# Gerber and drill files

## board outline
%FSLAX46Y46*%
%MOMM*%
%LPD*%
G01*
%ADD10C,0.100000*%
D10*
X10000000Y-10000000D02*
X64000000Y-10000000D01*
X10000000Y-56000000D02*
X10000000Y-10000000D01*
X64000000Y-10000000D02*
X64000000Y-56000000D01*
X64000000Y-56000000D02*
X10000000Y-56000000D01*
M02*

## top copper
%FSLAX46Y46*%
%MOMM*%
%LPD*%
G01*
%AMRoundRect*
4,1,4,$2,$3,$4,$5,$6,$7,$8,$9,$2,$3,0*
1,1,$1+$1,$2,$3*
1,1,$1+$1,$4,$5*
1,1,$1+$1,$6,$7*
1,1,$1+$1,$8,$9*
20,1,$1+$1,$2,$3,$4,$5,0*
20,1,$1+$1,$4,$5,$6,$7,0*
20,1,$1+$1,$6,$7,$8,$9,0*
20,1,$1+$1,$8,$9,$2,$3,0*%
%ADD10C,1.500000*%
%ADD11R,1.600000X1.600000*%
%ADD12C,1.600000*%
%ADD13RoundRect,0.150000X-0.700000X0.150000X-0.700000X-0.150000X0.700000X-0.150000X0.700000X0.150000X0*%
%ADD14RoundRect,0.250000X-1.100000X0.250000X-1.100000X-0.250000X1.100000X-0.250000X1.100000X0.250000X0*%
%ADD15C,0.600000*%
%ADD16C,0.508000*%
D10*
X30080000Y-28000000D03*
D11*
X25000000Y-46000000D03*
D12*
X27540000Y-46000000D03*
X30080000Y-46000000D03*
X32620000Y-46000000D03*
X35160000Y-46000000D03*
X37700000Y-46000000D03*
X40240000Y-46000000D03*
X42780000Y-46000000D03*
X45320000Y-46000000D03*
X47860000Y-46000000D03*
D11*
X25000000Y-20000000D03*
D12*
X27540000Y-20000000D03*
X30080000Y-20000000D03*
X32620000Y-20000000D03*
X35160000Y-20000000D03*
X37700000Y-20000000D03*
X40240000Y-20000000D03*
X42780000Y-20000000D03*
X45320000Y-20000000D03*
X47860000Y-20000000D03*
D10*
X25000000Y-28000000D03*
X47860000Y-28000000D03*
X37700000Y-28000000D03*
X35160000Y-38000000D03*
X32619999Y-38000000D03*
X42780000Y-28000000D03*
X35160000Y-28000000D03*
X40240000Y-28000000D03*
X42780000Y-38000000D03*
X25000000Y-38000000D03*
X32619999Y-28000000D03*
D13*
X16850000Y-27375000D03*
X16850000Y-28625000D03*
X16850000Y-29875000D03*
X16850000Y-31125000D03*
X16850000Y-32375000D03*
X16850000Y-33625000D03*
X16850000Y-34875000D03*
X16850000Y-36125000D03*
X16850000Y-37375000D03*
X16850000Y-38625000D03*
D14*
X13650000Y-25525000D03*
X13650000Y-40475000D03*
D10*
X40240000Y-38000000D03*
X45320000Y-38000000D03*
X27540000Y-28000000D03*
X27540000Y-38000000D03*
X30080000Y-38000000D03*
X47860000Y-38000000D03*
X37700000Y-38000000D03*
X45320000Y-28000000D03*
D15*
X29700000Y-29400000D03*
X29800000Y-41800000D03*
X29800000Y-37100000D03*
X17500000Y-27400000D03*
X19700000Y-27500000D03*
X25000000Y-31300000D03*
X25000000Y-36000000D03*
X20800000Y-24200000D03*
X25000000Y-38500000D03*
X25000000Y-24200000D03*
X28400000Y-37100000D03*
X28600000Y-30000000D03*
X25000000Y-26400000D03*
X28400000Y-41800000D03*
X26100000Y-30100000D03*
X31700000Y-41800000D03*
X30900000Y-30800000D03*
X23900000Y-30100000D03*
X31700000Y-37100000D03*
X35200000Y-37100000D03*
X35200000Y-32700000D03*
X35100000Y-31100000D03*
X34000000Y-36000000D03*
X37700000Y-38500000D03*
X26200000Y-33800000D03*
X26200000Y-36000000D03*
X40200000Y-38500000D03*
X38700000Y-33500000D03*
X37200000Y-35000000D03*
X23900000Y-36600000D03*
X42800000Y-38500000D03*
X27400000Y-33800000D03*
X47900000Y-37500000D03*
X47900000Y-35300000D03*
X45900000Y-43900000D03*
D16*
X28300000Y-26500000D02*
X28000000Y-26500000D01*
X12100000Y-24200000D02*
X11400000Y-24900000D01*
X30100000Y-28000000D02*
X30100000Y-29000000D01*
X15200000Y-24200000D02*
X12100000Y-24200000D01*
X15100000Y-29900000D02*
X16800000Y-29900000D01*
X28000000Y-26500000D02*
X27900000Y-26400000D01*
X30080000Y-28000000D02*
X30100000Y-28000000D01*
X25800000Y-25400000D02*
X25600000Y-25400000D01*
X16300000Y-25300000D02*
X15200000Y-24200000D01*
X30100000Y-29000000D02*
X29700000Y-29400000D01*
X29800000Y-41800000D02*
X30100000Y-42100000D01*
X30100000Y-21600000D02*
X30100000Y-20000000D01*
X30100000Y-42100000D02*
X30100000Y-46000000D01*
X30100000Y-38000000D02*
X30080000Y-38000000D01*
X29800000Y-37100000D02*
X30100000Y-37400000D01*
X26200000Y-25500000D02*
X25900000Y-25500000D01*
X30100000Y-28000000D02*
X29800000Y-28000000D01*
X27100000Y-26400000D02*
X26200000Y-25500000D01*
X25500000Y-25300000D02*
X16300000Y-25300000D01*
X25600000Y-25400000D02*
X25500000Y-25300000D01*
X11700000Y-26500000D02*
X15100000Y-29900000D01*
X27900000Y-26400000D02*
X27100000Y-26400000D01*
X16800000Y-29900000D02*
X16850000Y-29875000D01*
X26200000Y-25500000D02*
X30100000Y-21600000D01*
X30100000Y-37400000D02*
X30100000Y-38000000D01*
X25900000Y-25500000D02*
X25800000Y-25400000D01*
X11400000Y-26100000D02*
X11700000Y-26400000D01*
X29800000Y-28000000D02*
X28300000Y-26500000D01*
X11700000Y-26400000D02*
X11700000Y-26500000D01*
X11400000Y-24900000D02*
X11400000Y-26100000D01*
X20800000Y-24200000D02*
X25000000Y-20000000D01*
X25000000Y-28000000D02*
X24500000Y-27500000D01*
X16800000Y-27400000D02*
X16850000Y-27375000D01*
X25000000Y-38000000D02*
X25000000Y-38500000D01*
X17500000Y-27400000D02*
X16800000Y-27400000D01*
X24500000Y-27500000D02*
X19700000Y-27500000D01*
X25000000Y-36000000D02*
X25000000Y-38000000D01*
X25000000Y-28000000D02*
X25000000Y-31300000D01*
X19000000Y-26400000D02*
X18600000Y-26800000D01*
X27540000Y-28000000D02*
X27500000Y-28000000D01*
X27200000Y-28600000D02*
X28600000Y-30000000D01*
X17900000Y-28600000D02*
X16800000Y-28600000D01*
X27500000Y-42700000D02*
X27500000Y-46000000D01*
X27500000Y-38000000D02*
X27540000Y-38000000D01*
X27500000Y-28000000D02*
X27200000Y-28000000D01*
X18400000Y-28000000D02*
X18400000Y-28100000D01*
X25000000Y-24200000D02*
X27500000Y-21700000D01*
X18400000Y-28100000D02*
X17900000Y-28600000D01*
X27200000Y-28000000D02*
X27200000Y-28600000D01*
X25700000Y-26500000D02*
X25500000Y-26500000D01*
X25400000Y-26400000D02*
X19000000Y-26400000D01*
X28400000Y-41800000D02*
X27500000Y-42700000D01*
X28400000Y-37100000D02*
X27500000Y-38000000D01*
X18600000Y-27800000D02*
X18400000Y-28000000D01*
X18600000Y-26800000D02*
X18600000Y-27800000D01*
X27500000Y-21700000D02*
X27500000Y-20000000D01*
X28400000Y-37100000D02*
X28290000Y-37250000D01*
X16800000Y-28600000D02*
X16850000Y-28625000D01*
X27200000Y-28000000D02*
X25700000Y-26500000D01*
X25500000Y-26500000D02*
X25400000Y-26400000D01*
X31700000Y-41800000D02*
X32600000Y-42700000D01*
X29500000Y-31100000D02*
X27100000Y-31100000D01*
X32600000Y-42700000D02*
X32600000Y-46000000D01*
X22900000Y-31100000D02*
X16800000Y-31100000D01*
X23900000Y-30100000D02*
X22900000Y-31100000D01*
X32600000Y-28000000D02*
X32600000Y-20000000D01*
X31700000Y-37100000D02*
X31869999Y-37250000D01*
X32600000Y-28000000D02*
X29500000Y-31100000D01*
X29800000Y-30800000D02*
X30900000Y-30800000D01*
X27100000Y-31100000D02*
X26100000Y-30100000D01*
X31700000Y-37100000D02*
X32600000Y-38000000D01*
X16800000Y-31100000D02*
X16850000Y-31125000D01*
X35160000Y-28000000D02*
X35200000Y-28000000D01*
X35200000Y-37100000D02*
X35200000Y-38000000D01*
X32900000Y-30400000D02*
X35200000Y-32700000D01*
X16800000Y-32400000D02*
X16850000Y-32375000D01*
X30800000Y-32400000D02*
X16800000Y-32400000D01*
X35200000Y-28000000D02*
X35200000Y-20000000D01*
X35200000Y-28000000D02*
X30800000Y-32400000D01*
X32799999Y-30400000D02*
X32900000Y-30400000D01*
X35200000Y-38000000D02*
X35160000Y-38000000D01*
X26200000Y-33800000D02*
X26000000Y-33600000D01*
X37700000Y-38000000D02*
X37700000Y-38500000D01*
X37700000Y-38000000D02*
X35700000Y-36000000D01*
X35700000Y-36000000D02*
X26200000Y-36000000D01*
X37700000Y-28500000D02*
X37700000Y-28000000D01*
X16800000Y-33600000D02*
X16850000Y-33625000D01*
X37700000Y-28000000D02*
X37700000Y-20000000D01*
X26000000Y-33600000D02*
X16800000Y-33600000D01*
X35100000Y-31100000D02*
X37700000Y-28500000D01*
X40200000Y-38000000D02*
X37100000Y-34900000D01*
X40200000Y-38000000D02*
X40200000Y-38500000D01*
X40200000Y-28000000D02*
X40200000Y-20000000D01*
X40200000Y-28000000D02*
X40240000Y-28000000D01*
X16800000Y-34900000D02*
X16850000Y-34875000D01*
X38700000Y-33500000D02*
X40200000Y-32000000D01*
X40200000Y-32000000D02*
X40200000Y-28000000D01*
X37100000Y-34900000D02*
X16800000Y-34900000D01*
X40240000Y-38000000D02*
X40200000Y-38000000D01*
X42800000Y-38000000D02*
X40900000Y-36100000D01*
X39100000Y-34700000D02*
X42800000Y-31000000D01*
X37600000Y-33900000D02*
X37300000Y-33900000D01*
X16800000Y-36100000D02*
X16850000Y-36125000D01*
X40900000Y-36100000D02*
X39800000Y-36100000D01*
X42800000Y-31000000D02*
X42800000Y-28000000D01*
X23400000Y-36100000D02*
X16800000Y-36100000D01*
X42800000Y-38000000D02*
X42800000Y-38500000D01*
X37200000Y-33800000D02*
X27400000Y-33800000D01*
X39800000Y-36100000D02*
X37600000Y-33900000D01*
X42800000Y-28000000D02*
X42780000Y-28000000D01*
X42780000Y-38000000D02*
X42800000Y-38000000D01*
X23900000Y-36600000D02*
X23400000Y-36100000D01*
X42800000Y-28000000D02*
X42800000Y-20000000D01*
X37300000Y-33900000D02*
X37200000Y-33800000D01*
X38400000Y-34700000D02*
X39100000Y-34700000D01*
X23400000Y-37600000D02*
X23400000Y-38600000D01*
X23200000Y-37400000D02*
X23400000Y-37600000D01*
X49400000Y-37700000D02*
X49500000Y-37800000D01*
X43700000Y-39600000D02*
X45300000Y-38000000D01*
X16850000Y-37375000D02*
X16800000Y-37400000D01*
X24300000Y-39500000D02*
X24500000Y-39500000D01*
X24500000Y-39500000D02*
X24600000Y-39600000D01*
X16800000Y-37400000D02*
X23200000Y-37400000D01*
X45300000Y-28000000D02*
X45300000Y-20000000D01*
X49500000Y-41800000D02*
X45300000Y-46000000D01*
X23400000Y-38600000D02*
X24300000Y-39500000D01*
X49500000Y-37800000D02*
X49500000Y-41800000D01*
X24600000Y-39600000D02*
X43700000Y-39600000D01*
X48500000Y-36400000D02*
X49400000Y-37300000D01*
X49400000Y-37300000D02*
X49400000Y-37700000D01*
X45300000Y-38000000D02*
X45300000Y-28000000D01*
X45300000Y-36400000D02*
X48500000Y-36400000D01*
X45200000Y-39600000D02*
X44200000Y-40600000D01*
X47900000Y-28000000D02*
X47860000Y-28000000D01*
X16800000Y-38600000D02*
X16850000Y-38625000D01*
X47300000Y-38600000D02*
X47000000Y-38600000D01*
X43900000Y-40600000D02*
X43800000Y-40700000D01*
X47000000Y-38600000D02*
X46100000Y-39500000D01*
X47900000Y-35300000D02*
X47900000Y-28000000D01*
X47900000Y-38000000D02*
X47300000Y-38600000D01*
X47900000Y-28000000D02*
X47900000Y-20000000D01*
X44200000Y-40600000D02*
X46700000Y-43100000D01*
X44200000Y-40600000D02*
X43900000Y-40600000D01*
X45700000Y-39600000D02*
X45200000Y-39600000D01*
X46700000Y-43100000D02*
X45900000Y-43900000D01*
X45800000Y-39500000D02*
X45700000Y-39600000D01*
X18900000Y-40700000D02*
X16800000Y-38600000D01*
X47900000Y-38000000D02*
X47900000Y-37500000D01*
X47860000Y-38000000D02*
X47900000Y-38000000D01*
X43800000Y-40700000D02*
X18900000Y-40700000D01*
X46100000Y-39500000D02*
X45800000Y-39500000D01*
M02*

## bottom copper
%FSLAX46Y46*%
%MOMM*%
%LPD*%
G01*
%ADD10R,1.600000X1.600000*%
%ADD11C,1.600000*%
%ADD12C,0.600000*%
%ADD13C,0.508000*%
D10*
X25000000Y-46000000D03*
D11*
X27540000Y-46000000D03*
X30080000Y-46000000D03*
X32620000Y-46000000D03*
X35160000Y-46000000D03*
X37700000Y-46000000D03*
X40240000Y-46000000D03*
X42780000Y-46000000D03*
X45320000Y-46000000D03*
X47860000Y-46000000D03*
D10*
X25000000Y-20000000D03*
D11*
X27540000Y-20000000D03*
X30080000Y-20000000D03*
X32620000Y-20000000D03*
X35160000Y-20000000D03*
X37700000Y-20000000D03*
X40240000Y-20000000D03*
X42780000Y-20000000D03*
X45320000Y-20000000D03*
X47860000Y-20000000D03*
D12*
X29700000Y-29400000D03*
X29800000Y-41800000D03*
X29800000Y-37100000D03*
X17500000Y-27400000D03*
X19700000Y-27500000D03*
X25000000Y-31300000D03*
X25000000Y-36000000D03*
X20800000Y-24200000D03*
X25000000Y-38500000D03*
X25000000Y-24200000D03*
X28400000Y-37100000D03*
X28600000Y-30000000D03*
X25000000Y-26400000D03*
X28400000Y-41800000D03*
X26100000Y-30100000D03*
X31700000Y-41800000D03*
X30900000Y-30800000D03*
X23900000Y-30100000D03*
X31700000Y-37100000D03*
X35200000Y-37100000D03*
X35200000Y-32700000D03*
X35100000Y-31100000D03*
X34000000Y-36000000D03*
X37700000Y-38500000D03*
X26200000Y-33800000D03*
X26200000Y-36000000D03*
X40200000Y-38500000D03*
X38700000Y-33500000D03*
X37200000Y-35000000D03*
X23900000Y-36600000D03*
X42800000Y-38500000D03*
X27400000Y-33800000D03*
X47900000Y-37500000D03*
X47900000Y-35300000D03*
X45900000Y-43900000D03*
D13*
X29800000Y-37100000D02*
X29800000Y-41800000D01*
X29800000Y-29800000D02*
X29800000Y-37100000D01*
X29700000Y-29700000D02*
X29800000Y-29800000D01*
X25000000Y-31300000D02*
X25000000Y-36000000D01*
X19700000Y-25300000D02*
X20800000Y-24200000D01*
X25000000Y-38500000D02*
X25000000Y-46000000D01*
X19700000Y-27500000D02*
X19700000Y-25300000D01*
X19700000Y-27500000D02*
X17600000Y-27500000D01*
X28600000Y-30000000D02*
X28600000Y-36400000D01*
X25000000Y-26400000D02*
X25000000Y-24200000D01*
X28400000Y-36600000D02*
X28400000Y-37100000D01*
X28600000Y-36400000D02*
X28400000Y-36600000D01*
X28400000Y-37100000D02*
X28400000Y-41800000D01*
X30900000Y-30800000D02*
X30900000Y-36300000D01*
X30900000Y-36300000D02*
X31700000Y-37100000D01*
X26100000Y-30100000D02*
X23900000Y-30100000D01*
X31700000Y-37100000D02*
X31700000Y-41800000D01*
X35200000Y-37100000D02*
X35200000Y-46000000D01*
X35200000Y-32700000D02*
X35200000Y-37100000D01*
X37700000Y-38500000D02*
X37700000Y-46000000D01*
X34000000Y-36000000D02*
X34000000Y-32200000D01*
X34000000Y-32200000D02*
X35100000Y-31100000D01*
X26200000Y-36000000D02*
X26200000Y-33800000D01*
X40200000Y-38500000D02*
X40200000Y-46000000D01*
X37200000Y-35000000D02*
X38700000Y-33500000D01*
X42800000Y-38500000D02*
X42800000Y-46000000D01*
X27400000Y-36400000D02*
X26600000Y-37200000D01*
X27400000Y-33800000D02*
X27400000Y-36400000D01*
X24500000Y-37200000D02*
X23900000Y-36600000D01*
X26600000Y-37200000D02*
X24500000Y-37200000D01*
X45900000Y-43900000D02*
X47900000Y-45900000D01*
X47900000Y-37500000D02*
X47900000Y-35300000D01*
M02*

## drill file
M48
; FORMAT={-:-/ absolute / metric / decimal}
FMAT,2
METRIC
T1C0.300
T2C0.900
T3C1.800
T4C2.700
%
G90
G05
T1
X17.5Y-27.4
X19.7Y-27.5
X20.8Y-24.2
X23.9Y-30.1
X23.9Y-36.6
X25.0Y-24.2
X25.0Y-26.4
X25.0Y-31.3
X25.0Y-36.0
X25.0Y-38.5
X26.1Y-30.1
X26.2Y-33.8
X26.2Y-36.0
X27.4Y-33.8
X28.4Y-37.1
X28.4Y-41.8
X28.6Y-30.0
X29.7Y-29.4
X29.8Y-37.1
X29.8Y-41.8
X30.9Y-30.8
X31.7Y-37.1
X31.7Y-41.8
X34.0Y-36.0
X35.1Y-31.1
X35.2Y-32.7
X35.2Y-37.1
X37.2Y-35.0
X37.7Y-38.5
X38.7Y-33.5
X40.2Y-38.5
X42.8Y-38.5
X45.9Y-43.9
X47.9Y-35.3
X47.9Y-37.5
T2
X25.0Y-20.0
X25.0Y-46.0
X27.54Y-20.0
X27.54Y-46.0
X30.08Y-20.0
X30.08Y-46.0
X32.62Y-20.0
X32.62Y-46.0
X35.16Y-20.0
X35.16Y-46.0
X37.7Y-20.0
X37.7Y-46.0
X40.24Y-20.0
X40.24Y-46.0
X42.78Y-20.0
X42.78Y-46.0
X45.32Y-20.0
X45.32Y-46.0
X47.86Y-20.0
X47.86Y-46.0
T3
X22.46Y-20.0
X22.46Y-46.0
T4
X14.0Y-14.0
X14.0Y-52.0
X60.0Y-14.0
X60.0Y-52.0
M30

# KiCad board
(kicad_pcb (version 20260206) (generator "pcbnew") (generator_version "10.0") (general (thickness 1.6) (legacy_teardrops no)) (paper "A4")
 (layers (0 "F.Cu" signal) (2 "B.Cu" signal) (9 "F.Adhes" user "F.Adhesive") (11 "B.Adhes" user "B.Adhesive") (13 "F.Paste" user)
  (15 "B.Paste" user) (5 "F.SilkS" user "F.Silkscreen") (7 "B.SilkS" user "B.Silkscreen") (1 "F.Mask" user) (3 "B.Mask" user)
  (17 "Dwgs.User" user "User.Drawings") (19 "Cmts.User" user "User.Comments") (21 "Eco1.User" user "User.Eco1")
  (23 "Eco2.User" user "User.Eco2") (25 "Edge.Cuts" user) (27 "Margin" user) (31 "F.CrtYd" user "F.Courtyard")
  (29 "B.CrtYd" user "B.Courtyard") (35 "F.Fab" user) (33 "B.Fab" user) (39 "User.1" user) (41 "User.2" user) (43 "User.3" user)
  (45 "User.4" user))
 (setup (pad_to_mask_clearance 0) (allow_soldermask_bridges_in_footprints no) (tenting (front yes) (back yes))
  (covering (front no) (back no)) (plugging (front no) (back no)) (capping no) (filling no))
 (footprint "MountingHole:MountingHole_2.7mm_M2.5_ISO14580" (layer "F.Cu") (at 60 14)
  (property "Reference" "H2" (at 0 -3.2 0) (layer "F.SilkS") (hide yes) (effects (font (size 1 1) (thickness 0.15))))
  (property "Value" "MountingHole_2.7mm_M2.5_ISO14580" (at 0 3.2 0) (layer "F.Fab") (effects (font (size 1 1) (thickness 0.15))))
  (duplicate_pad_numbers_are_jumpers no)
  (pad "" np_thru_hole circle (at 0 0) (size 2.7 2.7) (drill 2.7) (layers "*.Cu" "*.Mask")))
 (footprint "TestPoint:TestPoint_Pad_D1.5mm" (layer "F.Cu") (at 30.08 28)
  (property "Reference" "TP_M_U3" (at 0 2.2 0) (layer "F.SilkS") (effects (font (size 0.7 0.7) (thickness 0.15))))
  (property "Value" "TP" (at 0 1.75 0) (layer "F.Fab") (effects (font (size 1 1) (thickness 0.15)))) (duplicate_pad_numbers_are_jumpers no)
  (pad "1" smd circle (at 0 0) (size 1.5 1.5) (layers "F.Cu" "F.Mask") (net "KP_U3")))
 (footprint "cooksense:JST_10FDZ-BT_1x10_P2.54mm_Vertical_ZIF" (layer "F.Cu") (at 25 46)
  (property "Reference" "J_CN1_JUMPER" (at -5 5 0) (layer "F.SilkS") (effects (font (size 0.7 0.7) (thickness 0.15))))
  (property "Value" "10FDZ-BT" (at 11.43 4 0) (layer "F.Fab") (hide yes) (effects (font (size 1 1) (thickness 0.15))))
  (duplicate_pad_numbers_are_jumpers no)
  (pad "" np_thru_hole circle (at -2.54 0) (size 1.8 1.8) (drill 1.8) (layers "*.Cu" "*.Mask"))
  (pad "1" thru_hole rect (at 0 0) (size 1.6 1.6) (drill 0.9) (layers "*.Cu" "*.Mask") (remove_unused_layers no) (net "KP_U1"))
  (pad "2" thru_hole circle (at 2.54 0) (size 1.6 1.6) (drill 0.9) (layers "*.Cu" "*.Mask") (remove_unused_layers no) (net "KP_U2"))
  (pad "3" thru_hole circle (at 5.08 0) (size 1.6 1.6) (drill 0.9) (layers "*.Cu" "*.Mask") (remove_unused_layers no) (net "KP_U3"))
  (pad "4" thru_hole circle (at 7.62 0) (size 1.6 1.6) (drill 0.9) (layers "*.Cu" "*.Mask") (remove_unused_layers no) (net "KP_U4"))
  (pad "5" thru_hole circle (at 10.16 0) (size 1.6 1.6) (drill 0.9) (layers "*.Cu" "*.Mask") (remove_unused_layers no) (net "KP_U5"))
  (pad "6" thru_hole circle (at 12.7 0) (size 1.6 1.6) (drill 0.9) (layers "*.Cu" "*.Mask") (remove_unused_layers no) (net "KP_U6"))
  (pad "7" thru_hole circle (at 15.24 0) (size 1.6 1.6) (drill 0.9) (layers "*.Cu" "*.Mask") (remove_unused_layers no) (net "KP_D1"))
  (pad "8" thru_hole circle (at 17.78 0) (size 1.6 1.6) (drill 0.9) (layers "*.Cu" "*.Mask") (remove_unused_layers no) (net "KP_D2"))
  (pad "9" thru_hole circle (at 20.32 0) (size 1.6 1.6) (drill 0.9) (layers "*.Cu" "*.Mask") (remove_unused_layers no) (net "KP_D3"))
  (pad "10" thru_hole circle (at 22.86 0) (size 1.6 1.6) (drill 0.9) (layers "*.Cu" "*.Mask") (remove_unused_layers no) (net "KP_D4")))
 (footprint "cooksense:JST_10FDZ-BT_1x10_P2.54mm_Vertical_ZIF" (layer "F.Cu") (at 25 20)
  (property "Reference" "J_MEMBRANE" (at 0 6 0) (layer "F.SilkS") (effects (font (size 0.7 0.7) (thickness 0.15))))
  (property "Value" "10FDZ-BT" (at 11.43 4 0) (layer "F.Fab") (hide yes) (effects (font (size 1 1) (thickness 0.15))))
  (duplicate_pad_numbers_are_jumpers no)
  (pad "" np_thru_hole circle (at -2.54 0) (size 1.8 1.8) (drill 1.8) (layers "*.Cu" "*.Mask"))
  (pad "1" thru_hole rect (at 0 0) (size 1.6 1.6) (drill 0.9) (layers "*.Cu" "*.Mask") (remove_unused_layers no) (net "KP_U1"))
  (pad "2" thru_hole circle (at 2.54 0) (size 1.6 1.6) (drill 0.9) (layers "*.Cu" "*.Mask") (remove_unused_layers no) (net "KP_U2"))
  (pad "3" thru_hole circle (at 5.08 0) (size 1.6 1.6) (drill 0.9) (layers "*.Cu" "*.Mask") (remove_unused_layers no) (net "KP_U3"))
  (pad "4" thru_hole circle (at 7.62 0) (size 1.6 1.6) (drill 0.9) (layers "*.Cu" "*.Mask") (remove_unused_layers no) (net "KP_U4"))
  (pad "5" thru_hole circle (at 10.16 0) (size 1.6 1.6) (drill 0.9) (layers "*.Cu" "*.Mask") (remove_unused_layers no) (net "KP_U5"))
  (pad "6" thru_hole circle (at 12.7 0) (size 1.6 1.6) (drill 0.9) (layers "*.Cu" "*.Mask") (remove_unused_layers no) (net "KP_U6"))
  (pad "7" thru_hole circle (at 15.24 0) (size 1.6 1.6) (drill 0.9) (layers "*.Cu" "*.Mask") (remove_unused_layers no) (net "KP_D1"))
  (pad "8" thru_hole circle (at 17.78 0) (size 1.6 1.6) (drill 0.9) (layers "*.Cu" "*.Mask") (remove_unused_layers no) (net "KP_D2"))
  (pad "9" thru_hole circle (at 20.32 0) (size 1.6 1.6) (drill 0.9) (layers "*.Cu" "*.Mask") (remove_unused_layers no) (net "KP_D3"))
  (pad "10" thru_hole circle (at 22.86 0) (size 1.6 1.6) (drill 0.9) (layers "*.Cu" "*.Mask") (remove_unused_layers no) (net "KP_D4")))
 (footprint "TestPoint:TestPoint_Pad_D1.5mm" (layer "F.Cu") (at 25 28)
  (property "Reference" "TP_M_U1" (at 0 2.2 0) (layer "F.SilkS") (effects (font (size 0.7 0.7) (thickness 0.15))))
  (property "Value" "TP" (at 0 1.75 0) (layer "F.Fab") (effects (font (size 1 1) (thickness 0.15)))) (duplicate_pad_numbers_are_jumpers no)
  (pad "1" smd circle (at 0 0) (size 1.5 1.5) (layers "F.Cu" "F.Mask") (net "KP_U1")))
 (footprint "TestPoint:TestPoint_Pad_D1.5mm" (layer "F.Cu") (at 47.86 28)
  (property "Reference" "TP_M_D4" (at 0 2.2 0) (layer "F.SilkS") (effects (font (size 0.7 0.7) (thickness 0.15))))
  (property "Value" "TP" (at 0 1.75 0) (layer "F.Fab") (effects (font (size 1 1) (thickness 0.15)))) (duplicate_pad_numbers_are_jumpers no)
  (pad "1" smd circle (at 0 0) (size 1.5 1.5) (layers "F.Cu" "F.Mask") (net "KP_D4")))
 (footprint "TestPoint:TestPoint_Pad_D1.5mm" (layer "F.Cu") (at 37.7 28)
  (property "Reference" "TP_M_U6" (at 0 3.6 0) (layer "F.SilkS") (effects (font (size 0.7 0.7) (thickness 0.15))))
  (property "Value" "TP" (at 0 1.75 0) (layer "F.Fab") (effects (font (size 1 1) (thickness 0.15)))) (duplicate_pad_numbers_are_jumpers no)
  (pad "1" smd circle (at 0 0) (size 1.5 1.5) (layers "F.Cu" "F.Mask") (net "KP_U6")))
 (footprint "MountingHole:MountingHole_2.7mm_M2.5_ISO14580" (layer "F.Cu") (at 60 52)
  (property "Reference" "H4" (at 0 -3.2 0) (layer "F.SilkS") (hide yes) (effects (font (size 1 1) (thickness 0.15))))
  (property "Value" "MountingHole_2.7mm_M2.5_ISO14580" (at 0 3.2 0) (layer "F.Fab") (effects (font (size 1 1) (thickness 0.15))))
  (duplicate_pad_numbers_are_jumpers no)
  (pad "" np_thru_hole circle (at 0 0) (size 2.7 2.7) (drill 2.7) (layers "*.Cu" "*.Mask")))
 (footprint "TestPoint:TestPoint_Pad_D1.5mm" (layer "F.Cu") (at 35.16 38)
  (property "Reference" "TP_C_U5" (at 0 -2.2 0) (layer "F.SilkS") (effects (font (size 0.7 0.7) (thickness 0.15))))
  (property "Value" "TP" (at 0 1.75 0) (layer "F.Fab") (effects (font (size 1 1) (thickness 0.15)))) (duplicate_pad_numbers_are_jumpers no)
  (pad "1" smd circle (at 0 0) (size 1.5 1.5) (layers "F.Cu" "F.Mask") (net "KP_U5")))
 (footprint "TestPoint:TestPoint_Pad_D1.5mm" (layer "F.Cu") (at 32.619999 38)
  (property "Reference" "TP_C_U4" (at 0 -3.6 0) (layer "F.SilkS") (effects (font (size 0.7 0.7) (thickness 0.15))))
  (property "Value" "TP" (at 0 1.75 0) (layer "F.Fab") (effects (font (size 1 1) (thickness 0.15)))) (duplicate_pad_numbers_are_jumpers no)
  (pad "1" smd circle (at 0 0) (size 1.5 1.5) (layers "F.Cu" "F.Mask") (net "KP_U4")))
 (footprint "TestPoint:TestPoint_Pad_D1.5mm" (layer "F.Cu") (at 42.78 28)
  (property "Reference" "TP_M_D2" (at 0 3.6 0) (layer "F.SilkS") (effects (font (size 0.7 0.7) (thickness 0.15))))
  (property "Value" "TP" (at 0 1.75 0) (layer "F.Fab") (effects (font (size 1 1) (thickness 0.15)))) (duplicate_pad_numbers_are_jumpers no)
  (pad "1" smd circle (at 0 0) (size 1.5 1.5) (layers "F.Cu" "F.Mask") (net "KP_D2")))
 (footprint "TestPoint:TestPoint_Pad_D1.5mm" (layer "F.Cu") (at 35.16 28)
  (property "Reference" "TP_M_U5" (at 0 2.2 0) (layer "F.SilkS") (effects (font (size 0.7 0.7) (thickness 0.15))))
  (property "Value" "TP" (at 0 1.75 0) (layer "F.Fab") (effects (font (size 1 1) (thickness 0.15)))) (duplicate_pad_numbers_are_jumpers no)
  (pad "1" smd circle (at 0 0) (size 1.5 1.5) (layers "F.Cu" "F.Mask") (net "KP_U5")))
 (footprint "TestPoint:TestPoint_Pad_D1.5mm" (layer "F.Cu") (at 40.24 28)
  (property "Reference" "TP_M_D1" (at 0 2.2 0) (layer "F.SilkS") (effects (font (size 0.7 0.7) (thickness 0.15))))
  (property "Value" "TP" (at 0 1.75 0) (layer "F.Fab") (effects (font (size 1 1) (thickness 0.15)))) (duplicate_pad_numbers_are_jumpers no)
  (pad "1" smd circle (at 0 0) (size 1.5 1.5) (layers "F.Cu" "F.Mask") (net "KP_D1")))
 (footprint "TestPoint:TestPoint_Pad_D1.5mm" (layer "F.Cu") (at 42.78 38)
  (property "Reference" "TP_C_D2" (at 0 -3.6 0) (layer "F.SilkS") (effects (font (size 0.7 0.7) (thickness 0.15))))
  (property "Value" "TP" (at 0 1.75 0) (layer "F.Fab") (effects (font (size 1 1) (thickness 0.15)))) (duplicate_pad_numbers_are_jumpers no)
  (pad "1" smd circle (at 0 0) (size 1.5 1.5) (layers "F.Cu" "F.Mask") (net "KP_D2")))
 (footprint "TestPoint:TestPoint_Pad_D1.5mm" (layer "F.Cu") (at 25 38)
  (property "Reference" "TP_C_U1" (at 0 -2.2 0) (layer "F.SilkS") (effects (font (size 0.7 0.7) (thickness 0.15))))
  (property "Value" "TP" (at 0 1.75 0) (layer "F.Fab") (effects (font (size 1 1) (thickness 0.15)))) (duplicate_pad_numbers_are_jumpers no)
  (pad "1" smd circle (at 0 0) (size 1.5 1.5) (layers "F.Cu" "F.Mask") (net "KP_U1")))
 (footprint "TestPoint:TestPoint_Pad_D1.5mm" (layer "F.Cu") (at 32.619999 28)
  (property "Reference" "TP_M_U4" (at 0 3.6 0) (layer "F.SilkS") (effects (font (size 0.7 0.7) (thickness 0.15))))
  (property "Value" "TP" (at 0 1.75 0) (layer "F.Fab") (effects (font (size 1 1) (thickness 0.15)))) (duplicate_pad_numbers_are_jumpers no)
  (pad "1" smd circle (at 0 0) (size 1.5 1.5) (layers "F.Cu" "F.Mask") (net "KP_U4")))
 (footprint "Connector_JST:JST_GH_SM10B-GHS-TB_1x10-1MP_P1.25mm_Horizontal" (layer "F.Cu") (at 15 33 -90)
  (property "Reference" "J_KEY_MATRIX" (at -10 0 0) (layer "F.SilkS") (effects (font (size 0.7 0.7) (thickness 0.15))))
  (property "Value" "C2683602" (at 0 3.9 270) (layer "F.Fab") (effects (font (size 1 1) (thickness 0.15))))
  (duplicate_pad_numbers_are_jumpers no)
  (pad "1" smd roundrect (at -5.625 -1.85 270) (size 0.6 1.7) (layers "F.Cu" "F.Mask" "F.Paste") (roundrect_rratio 0.25) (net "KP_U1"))
  (pad "2" smd roundrect (at -4.375 -1.85 270) (size 0.6 1.7) (layers "F.Cu" "F.Mask" "F.Paste") (roundrect_rratio 0.25) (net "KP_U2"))
  (pad "3" smd roundrect (at -3.125 -1.85 270) (size 0.6 1.7) (layers "F.Cu" "F.Mask" "F.Paste") (roundrect_rratio 0.25) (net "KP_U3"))
  (pad "4" smd roundrect (at -1.875 -1.85 270) (size 0.6 1.7) (layers "F.Cu" "F.Mask" "F.Paste") (roundrect_rratio 0.25) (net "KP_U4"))
  (pad "5" smd roundrect (at -0.625 -1.85 270) (size 0.6 1.7) (layers "F.Cu" "F.Mask" "F.Paste") (roundrect_rratio 0.25) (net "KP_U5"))
  (pad "6" smd roundrect (at 0.625 -1.85 270) (size 0.6 1.7) (layers "F.Cu" "F.Mask" "F.Paste") (roundrect_rratio 0.25) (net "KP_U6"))
  (pad "7" smd roundrect (at 1.875 -1.85 270) (size 0.6 1.7) (layers "F.Cu" "F.Mask" "F.Paste") (roundrect_rratio 0.25) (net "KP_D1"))
  (pad "8" smd roundrect (at 3.125 -1.85 270) (size 0.6 1.7) (layers "F.Cu" "F.Mask" "F.Paste") (roundrect_rratio 0.25) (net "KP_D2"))
  (pad "9" smd roundrect (at 4.375 -1.85 270) (size 0.6 1.7) (layers "F.Cu" "F.Mask" "F.Paste") (roundrect_rratio 0.25) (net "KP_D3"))
  (pad "10" smd roundrect (at 5.625 -1.85 270) (size 0.6 1.7) (layers "F.Cu" "F.Mask" "F.Paste") (roundrect_rratio 0.25) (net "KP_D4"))
  (pad "MP" smd roundrect (at -7.475 1.35 270) (size 1 2.7) (layers "F.Cu" "F.Mask" "F.Paste") (roundrect_rratio 0.25))
  (pad "MP" smd roundrect (at 7.475 1.35 270) (size 1 2.7) (layers "F.Cu" "F.Mask" "F.Paste") (roundrect_rratio 0.25)))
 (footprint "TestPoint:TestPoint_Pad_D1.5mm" (layer "F.Cu") (at 40.24 38)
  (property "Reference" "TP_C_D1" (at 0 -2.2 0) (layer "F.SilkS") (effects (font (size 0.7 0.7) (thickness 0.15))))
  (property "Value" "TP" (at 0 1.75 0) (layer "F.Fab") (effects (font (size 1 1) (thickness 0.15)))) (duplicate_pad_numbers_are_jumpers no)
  (pad "1" smd circle (at 0 0) (size 1.5 1.5) (layers "F.Cu" "F.Mask") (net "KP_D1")))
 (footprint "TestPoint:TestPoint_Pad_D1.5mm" (layer "F.Cu") (at 45.32 38)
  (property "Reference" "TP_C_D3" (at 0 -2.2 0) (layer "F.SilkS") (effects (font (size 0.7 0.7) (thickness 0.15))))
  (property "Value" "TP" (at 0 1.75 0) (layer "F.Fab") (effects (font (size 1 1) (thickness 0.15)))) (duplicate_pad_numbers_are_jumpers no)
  (pad "1" smd circle (at 0 0) (size 1.5 1.5) (layers "F.Cu" "F.Mask") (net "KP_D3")))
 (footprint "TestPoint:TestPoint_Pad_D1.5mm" (layer "F.Cu") (at 27.54 28)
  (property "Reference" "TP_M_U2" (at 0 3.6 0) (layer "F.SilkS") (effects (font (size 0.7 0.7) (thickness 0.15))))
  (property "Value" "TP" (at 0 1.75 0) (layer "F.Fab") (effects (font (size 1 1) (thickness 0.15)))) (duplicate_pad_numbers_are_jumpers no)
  (pad "1" smd circle (at 0 0) (size 1.5 1.5) (layers "F.Cu" "F.Mask") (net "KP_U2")))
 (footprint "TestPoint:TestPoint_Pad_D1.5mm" (layer "F.Cu") (at 27.54 38)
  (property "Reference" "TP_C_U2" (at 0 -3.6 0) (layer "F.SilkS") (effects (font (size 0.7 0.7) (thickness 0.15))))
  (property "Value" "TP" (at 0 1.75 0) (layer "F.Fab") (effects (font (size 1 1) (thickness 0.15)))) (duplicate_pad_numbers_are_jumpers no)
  (pad "1" smd circle (at 0 0) (size 1.5 1.5) (layers "F.Cu" "F.Mask") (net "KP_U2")))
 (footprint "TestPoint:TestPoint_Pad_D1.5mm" (layer "F.Cu") (at 30.08 38)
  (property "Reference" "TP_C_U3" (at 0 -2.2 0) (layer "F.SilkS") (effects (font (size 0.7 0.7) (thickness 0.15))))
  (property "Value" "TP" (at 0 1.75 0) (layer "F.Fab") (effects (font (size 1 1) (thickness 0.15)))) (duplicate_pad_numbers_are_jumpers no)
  (pad "1" smd circle (at 0 0) (size 1.5 1.5) (layers "F.Cu" "F.Mask") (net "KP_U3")))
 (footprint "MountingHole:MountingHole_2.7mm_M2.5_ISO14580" (layer "F.Cu") (at 14 52)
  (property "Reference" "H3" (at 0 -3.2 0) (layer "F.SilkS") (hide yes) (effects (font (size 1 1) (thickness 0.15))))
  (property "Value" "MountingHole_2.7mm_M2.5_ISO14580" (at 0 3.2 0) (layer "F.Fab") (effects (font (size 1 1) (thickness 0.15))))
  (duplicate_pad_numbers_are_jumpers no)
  (pad "" np_thru_hole circle (at 0 0) (size 2.7 2.7) (drill 2.7) (layers "*.Cu" "*.Mask")))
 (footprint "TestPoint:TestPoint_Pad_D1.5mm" (layer "F.Cu") (at 47.86 38)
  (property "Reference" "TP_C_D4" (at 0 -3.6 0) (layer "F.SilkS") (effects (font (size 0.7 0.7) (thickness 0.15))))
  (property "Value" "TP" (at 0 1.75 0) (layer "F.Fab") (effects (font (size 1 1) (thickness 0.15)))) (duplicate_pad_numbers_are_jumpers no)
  (pad "1" smd circle (at 0 0) (size 1.5 1.5) (layers "F.Cu" "F.Mask") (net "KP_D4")))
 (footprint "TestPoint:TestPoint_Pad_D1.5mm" (layer "F.Cu") (at 37.7 38)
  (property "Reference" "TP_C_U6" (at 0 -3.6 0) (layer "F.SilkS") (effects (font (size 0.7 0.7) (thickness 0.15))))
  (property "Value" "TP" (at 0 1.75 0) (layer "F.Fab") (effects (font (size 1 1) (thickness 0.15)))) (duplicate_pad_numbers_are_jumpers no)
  (pad "1" smd circle (at 0 0) (size 1.5 1.5) (layers "F.Cu" "F.Mask") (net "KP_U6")))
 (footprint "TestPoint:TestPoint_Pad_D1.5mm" (layer "F.Cu") (at 45.32 28)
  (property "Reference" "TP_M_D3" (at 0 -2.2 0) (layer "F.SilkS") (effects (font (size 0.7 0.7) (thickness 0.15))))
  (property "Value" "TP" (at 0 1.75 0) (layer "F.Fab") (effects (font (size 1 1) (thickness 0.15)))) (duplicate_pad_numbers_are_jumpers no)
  (pad "1" smd circle (at 0 0) (size 1.5 1.5) (layers "F.Cu" "F.Mask") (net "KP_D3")))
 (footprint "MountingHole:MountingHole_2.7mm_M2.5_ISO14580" (layer "F.Cu") (at 14 14)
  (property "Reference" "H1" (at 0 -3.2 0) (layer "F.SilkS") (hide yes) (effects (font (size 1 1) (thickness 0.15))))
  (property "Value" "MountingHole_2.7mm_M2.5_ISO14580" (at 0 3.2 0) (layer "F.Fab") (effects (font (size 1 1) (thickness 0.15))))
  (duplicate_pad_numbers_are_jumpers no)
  (pad "" np_thru_hole circle (at 0 0) (size 2.7 2.7) (drill 2.7) (layers "*.Cu" "*.Mask")))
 (gr_line (start 10 10) (end 64 10) (stroke (width 0.1) (type default)) (layer "Edge.Cuts"))
 (gr_line (start 10 56) (end 10 10) (stroke (width 0.1) (type default)) (layer "Edge.Cuts"))
 (gr_line (start 64 10) (end 64 56) (stroke (width 0.1) (type default)) (layer "Edge.Cuts"))
 (gr_line (start 64 56) (end 10 56) (stroke (width 0.1) (type default)) (layer "Edge.Cuts"))
 (segment (start 28.3 26.5) (end 28 26.5) (width 0.508) (layer "F.Cu") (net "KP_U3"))
 (segment (start 12.1 24.2) (end 11.4 24.9) (width 0.508) (layer "F.Cu") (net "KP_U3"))
 (segment (start 30.1 28) (end 30.1 29) (width 0.508) (layer "F.Cu") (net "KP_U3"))
 (segment (start 15.2 24.2) (end 12.1 24.2) (width 0.508) (layer "F.Cu") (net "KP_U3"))
 (segment (start 15.1 29.9) (end 16.8 29.9) (width 0.508) (layer "F.Cu") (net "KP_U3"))
 (segment (start 28 26.5) (end 27.9 26.4) (width 0.508) (layer "F.Cu") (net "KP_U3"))
 (segment (start 30.08 28) (end 30.1 28) (width 0.508) (layer "F.Cu") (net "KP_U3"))
 (segment (start 25.8 25.4) (end 25.6 25.4) (width 0.508) (layer "F.Cu") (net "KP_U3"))
 (segment (start 16.3 25.3) (end 15.2 24.2) (width 0.508) (layer "F.Cu") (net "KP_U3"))
 (segment (start 30.1 29) (end 29.7 29.4) (width 0.508) (layer "F.Cu") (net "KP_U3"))
 (segment (start 29.8 41.8) (end 30.1 42.1) (width 0.508) (layer "F.Cu") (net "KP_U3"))
 (segment (start 30.1 21.6) (end 30.1 20) (width 0.508) (layer "F.Cu") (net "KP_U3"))
 (segment (start 30.1 42.1) (end 30.1 46) (width 0.508) (layer "F.Cu") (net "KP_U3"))
 (segment (start 30.1 38) (end 30.08 38) (width 0.508) (layer "F.Cu") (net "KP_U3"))
 (segment (start 29.8 37.1) (end 30.1 37.4) (width 0.508) (layer "F.Cu") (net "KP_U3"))
 (segment (start 26.2 25.5) (end 25.9 25.5) (width 0.508) (layer "F.Cu") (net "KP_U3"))
 (segment (start 30.1 28) (end 29.8 28) (width 0.508) (layer "F.Cu") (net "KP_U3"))
 (segment (start 27.1 26.4) (end 26.2 25.5) (width 0.508) (layer "F.Cu") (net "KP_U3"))
 (segment (start 25.5 25.3) (end 16.3 25.3) (width 0.508) (layer "F.Cu") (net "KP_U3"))
 (segment (start 25.6 25.4) (end 25.5 25.3) (width 0.508) (layer "F.Cu") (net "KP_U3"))
 (segment (start 11.7 26.5) (end 15.1 29.9) (width 0.508) (layer "F.Cu") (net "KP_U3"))
 (segment (start 27.9 26.4) (end 27.1 26.4) (width 0.508) (layer "F.Cu") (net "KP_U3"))
 (segment (start 16.8 29.9) (end 16.85 29.875) (width 0.508) (layer "F.Cu") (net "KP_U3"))
 (segment (start 26.2 25.5) (end 30.1 21.6) (width 0.508) (layer "F.Cu") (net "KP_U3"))
 (segment (start 30.1 37.4) (end 30.1 38) (width 0.508) (layer "F.Cu") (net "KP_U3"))
 (segment (start 25.9 25.5) (end 25.8 25.4) (width 0.508) (layer "F.Cu") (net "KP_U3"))
 (segment (start 11.4 26.1) (end 11.7 26.4) (width 0.508) (layer "F.Cu") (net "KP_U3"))
 (segment (start 29.8 28) (end 28.3 26.5) (width 0.508) (layer "F.Cu") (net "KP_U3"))
 (segment (start 11.7 26.4) (end 11.7 26.5) (width 0.508) (layer "F.Cu") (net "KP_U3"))
 (segment (start 11.4 24.9) (end 11.4 26.1) (width 0.508) (layer "F.Cu") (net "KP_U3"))
 (via (at 29.7 29.4) (size 0.6) (drill 0.3) (layers "F.Cu" "B.Cu") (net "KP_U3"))
 (via (at 29.8 41.8) (size 0.6) (drill 0.3) (layers "F.Cu" "B.Cu") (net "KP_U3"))
 (via (at 29.8 37.1) (size 0.6) (drill 0.3) (layers "F.Cu" "B.Cu") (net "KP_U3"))
 (segment (start 29.8 37.1) (end 29.8 41.8) (width 0.508) (layer "B.Cu") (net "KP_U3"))
 (segment (start 29.8 29.8) (end 29.8 37.1) (width 0.508) (layer "B.Cu") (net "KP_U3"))
 (segment (start 29.7 29.7) (end 29.8 29.8) (width 0.508) (layer "B.Cu") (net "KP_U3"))
 (segment (start 20.8 24.2) (end 25 20) (width 0.508) (layer "F.Cu") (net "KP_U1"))
 (segment (start 25 28) (end 24.5 27.5) (width 0.508) (layer "F.Cu") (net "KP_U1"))
 (segment (start 16.8 27.4) (end 16.85 27.375) (width 0.508) (layer "F.Cu") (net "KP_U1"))
 (segment (start 25 38) (end 25 38.5) (width 0.508) (layer "F.Cu") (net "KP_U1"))
 (segment (start 17.5 27.4) (end 16.8 27.4) (width 0.508) (layer "F.Cu") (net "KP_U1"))
 (segment (start 24.5 27.5) (end 19.7 27.5) (width 0.508) (layer "F.Cu") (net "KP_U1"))
 (segment (start 25 36) (end 25 38) (width 0.508) (layer "F.Cu") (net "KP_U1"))
 (segment (start 25 28) (end 25 31.3) (width 0.508) (layer "F.Cu") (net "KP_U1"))
 (via (at 17.5 27.4) (size 0.6) (drill 0.3) (layers "F.Cu" "B.Cu") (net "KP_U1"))
 (via (at 19.7 27.5) (size 0.6) (drill 0.3) (layers "F.Cu" "B.Cu") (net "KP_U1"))
 (via (at 25 31.3) (size 0.6) (drill 0.3) (layers "F.Cu" "B.Cu") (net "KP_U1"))
 (via (at 25 36) (size 0.6) (drill 0.3) (layers "F.Cu" "B.Cu") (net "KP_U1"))
 (via (at 20.8 24.2) (size 0.6) (drill 0.3) (layers "F.Cu" "B.Cu") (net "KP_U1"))
 (via (at 25 38.5) (size 0.6) (drill 0.3) (layers "F.Cu" "B.Cu") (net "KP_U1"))
 (segment (start 25 31.3) (end 25 36) (width 0.508) (layer "B.Cu") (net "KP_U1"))
 (segment (start 19.7 25.3) (end 20.8 24.2) (width 0.508) (layer "B.Cu") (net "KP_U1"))
 (segment (start 25 38.5) (end 25 46) (width 0.508) (layer "B.Cu") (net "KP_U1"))
 (segment (start 19.7 27.5) (end 19.7 25.3) (width 0.508) (layer "B.Cu") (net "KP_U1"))
 (segment (start 19.7 27.5) (end 17.6 27.5) (width 0.508) (layer "B.Cu") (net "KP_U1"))
 (segment (start 19 26.4) (end 18.6 26.8) (width 0.508) (layer "F.Cu") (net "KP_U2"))
 (segment (start 27.54 28) (end 27.5 28) (width 0.508) (layer "F.Cu") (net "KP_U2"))
 (segment (start 27.2 28.6) (end 28.6 30) (width 0.508) (layer "F.Cu") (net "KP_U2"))
 (segment (start 17.9 28.6) (end 16.8 28.6) (width 0.508) (layer "F.Cu") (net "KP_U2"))
 (segment (start 27.5 42.7) (end 27.5 46) (width 0.508) (layer "F.Cu") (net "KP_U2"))
 (segment (start 27.5 38) (end 27.54 38) (width 0.508) (layer "F.Cu") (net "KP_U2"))
 (segment (start 27.5 28) (end 27.2 28) (width 0.508) (layer "F.Cu") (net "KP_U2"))
 (segment (start 18.4 28) (end 18.4 28.1) (width 0.508) (layer "F.Cu") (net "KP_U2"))
 (segment (start 25 24.2) (end 27.5 21.7) (width 0.508) (layer "F.Cu") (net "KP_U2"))
 (segment (start 18.4 28.1) (end 17.9 28.6) (width 0.508) (layer "F.Cu") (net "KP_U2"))
 (segment (start 27.2 28) (end 27.2 28.6) (width 0.508) (layer "F.Cu") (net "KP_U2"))
 (segment (start 25.7 26.5) (end 25.5 26.5) (width 0.508) (layer "F.Cu") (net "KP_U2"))
 (segment (start 25.4 26.4) (end 19 26.4) (width 0.508) (layer "F.Cu") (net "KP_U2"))
 (segment (start 28.4 41.8) (end 27.5 42.7) (width 0.508) (layer "F.Cu") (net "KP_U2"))
 (segment (start 28.4 37.1) (end 27.5 38) (width 0.508) (layer "F.Cu") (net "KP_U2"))
 (segment (start 18.6 27.8) (end 18.4 28) (width 0.508) (layer "F.Cu") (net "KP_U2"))
 (segment (start 18.6 26.8) (end 18.6 27.8) (width 0.508) (layer "F.Cu") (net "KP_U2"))
 (segment (start 27.5 21.7) (end 27.5 20) (width 0.508) (layer "F.Cu") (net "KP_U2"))
 (segment (start 28.4 37.1) (end 28.29 37.25) (width 0.508) (layer "F.Cu") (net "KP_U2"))
 (segment (start 16.8 28.6) (end 16.85 28.625) (width 0.508) (layer "F.Cu") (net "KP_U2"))
 (segment (start 27.2 28) (end 25.7 26.5) (width 0.508) (layer "F.Cu") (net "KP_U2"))
 (segment (start 25.5 26.5) (end 25.4 26.4) (width 0.508) (layer "F.Cu") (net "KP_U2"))
 (via (at 25 24.2) (size 0.6) (drill 0.3) (layers "F.Cu" "B.Cu") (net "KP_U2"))
 (via (at 28.4 37.1) (size 0.6) (drill 0.3) (layers "F.Cu" "B.Cu") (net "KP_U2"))
 (via (at 28.6 30) (size 0.6) (drill 0.3) (layers "F.Cu" "B.Cu") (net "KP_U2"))
 (via (at 25 26.4) (size 0.6) (drill 0.3) (layers "F.Cu" "B.Cu") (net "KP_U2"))
 (via (at 28.4 41.8) (size 0.6) (drill 0.3) (layers "F.Cu" "B.Cu") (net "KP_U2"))
 (segment (start 28.6 30) (end 28.6 36.4) (width 0.508) (layer "B.Cu") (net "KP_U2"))
 (segment (start 25 26.4) (end 25 24.2) (width 0.508) (layer "B.Cu") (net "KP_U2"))
 (segment (start 28.4 36.6) (end 28.4 37.1) (width 0.508) (layer "B.Cu") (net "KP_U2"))
 (segment (start 28.6 36.4) (end 28.4 36.6) (width 0.508) (layer "B.Cu") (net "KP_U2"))
 (segment (start 28.4 37.1) (end 28.4 41.8) (width 0.508) (layer "B.Cu") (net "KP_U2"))
 (segment (start 31.7 41.8) (end 32.6 42.7) (width 0.508) (layer "F.Cu") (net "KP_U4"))
 (segment (start 29.5 31.1) (end 27.1 31.1) (width 0.508) (layer "F.Cu") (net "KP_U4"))
 (segment (start 32.6 42.7) (end 32.6 46) (width 0.508) (layer "F.Cu") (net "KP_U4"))
 (segment (start 22.9 31.1) (end 16.8 31.1) (width 0.508) (layer "F.Cu") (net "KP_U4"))
 (segment (start 23.9 30.1) (end 22.9 31.1) (width 0.508) (layer "F.Cu") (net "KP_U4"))
 (segment (start 32.6 28) (end 32.6 20) (width 0.508) (layer "F.Cu") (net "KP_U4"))
 (segment (start 31.7 37.1) (end 31.869999 37.25) (width 0.508) (layer "F.Cu") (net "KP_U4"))
 (segment (start 32.6 28) (end 29.5 31.1) (width 0.508) (layer "F.Cu") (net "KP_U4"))
 (segment (start 29.8 30.8) (end 30.9 30.8) (width 0.508) (layer "F.Cu") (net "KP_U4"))
 (segment (start 27.1 31.1) (end 26.1 30.1) (width 0.508) (layer "F.Cu") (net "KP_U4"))
 (segment (start 31.7 37.1) (end 32.6 38) (width 0.508) (layer "F.Cu") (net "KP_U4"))
 (segment (start 16.8 31.1) (end 16.85 31.125) (width 0.508) (layer "F.Cu") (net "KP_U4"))
 (via (at 26.1 30.1) (size 0.6) (drill 0.3) (layers "F.Cu" "B.Cu") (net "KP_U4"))
 (via (at 31.7 41.8) (size 0.6) (drill 0.3) (layers "F.Cu" "B.Cu") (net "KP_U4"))
 (via (at 30.9 30.8) (size 0.6) (drill 0.3) (layers "F.Cu" "B.Cu") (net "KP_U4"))
 (via (at 23.9 30.1) (size 0.6) (drill 0.3) (layers "F.Cu" "B.Cu") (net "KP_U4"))
 (via (at 31.7 37.1) (size 0.6) (drill 0.3) (layers "F.Cu" "B.Cu") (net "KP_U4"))
 (segment (start 30.9 30.8) (end 30.9 36.3) (width 0.508) (layer "B.Cu") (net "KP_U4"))
 (segment (start 30.9 36.3) (end 31.7 37.1) (width 0.508) (layer "B.Cu") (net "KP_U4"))
 (segment (start 26.1 30.1) (end 23.9 30.1) (width 0.508) (layer "B.Cu") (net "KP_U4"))
 (segment (start 31.7 37.1) (end 31.7 41.8) (width 0.508) (layer "B.Cu") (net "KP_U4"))
 (segment (start 35.16 28) (end 35.2 28) (width 0.508) (layer "F.Cu") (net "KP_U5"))
 (segment (start 35.2 37.1) (end 35.2 38) (width 0.508) (layer "F.Cu") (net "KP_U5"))
 (segment (start 32.9 30.4) (end 35.2 32.7) (width 0.508) (layer "F.Cu") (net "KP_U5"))
 (segment (start 16.8 32.4) (end 16.85 32.375) (width 0.508) (layer "F.Cu") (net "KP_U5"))
 (segment (start 30.8 32.4) (end 16.8 32.4) (width 0.508) (layer "F.Cu") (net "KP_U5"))
 (segment (start 35.2 28) (end 35.2 20) (width 0.508) (layer "F.Cu") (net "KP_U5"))
 (segment (start 35.2 28) (end 30.8 32.4) (width 0.508) (layer "F.Cu") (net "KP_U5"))
 (segment (start 32.799999 30.4) (end 32.9 30.4) (width 0.508) (layer "F.Cu") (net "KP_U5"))
 (segment (start 35.2 38) (end 35.16 38) (width 0.508) (layer "F.Cu") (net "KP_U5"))
 (via (at 35.2 37.1) (size 0.6) (drill 0.3) (layers "F.Cu" "B.Cu") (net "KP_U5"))
 (via (at 35.2 32.7) (size 0.6) (drill 0.3) (layers "F.Cu" "B.Cu") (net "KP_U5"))
 (segment (start 35.2 37.1) (end 35.2 46) (width 0.508) (layer "B.Cu") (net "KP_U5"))
 (segment (start 35.2 32.7) (end 35.2 37.1) (width 0.508) (layer "B.Cu") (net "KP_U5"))
 (segment (start 26.2 33.8) (end 26 33.6) (width 0.508) (layer "F.Cu") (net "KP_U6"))
 (segment (start 37.7 38) (end 37.7 38.5) (width 0.508) (layer "F.Cu") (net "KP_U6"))
 (segment (start 37.7 38) (end 35.7 36) (width 0.508) (layer "F.Cu") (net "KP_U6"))
 (segment (start 35.7 36) (end 26.2 36) (width 0.508) (layer "F.Cu") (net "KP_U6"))
 (segment (start 37.7 28.5) (end 37.7 28) (width 0.508) (layer "F.Cu") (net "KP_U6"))
 (segment (start 16.8 33.6) (end 16.85 33.625) (width 0.508) (layer "F.Cu") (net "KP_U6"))
 (segment (start 37.7 28) (end 37.7 20) (width 0.508) (layer "F.Cu") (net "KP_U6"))
 (segment (start 26 33.6) (end 16.8 33.6) (width 0.508) (layer "F.Cu") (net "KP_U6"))
 (segment (start 35.1 31.1) (end 37.7 28.5) (width 0.508) (layer "F.Cu") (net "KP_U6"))
 (via (at 35.1 31.1) (size 0.6) (drill 0.3) (layers "F.Cu" "B.Cu") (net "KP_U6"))
 (via (at 34 36) (size 0.6) (drill 0.3) (layers "F.Cu" "B.Cu") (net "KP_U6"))
 (via (at 37.7 38.5) (size 0.6) (drill 0.3) (layers "F.Cu" "B.Cu") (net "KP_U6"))
 (via (at 26.2 33.8) (size 0.6) (drill 0.3) (layers "F.Cu" "B.Cu") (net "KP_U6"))
 (via (at 26.2 36) (size 0.6) (drill 0.3) (layers "F.Cu" "B.Cu") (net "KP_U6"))
 (segment (start 37.7 38.5) (end 37.7 46) (width 0.508) (layer "B.Cu") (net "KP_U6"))
 (segment (start 34 36) (end 34 32.2) (width 0.508) (layer "B.Cu") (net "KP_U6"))
 (segment (start 34 32.2) (end 35.1 31.1) (width 0.508) (layer "B.Cu") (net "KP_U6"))
 (segment (start 26.2 36) (end 26.2 33.8) (width 0.508) (layer "B.Cu") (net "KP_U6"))
 (segment (start 40.2 38) (end 37.1 34.9) (width 0.508) (layer "F.Cu") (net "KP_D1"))
 (segment (start 40.2 38) (end 40.2 38.5) (width 0.508) (layer "F.Cu") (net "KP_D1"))
 (segment (start 40.2 28) (end 40.2 20) (width 0.508) (layer "F.Cu") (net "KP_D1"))
 (segment (start 40.2 28) (end 40.24 28) (width 0.508) (layer "F.Cu") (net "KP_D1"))
 (segment (start 16.8 34.9) (end 16.85 34.875) (width 0.508) (layer "F.Cu") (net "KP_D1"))
 (segment (start 38.7 33.5) (end 40.2 32) (width 0.508) (layer "F.Cu") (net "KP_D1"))
 (segment (start 40.2 32) (end 40.2 28) (width 0.508) (layer "F.Cu") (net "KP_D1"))
 (segment (start 37.1 34.9) (end 16.8 34.9) (width 0.508) (layer "F.Cu") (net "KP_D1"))
 (segment (start 40.24 38) (end 40.2 38) (width 0.508) (layer "F.Cu") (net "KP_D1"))
 (via (at 40.2 38.5) (size 0.6) (drill 0.3) (layers "F.Cu" "B.Cu") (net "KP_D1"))
 (via (at 38.7 33.5) (size 0.6) (drill 0.3) (layers "F.Cu" "B.Cu") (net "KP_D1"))
 (via (at 37.2 35) (size 0.6) (drill 0.3) (layers "F.Cu" "B.Cu") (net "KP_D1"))
 (segment (start 40.2 38.5) (end 40.2 46) (width 0.508) (layer "B.Cu") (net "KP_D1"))
 (segment (start 37.2 35) (end 38.7 33.5) (width 0.508) (layer "B.Cu") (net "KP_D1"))
 (segment (start 42.8 38) (end 40.9 36.1) (width 0.508) (layer "F.Cu") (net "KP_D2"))
 (segment (start 39.1 34.7) (end 42.8 31) (width 0.508) (layer "F.Cu") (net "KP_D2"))
 (segment (start 37.6 33.9) (end 37.3 33.9) (width 0.508) (layer "F.Cu") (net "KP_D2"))
 (segment (start 16.8 36.1) (end 16.85 36.125) (width 0.508) (layer "F.Cu") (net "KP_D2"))
 (segment (start 40.9 36.1) (end 39.8 36.1) (width 0.508) (layer "F.Cu") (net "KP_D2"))
 (segment (start 42.8 31) (end 42.8 28) (width 0.508) (layer "F.Cu") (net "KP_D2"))
 (segment (start 23.4 36.1) (end 16.8 36.1) (width 0.508) (layer "F.Cu") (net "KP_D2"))
 (segment (start 42.8 38) (end 42.8 38.5) (width 0.508) (layer "F.Cu") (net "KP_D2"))
 (segment (start 37.2 33.8) (end 27.4 33.8) (width 0.508) (layer "F.Cu") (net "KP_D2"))
 (segment (start 39.8 36.1) (end 37.6 33.9) (width 0.508) (layer "F.Cu") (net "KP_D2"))
 (segment (start 42.8 28) (end 42.78 28) (width 0.508) (layer "F.Cu") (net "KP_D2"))
 (segment (start 42.78 38) (end 42.8 38) (width 0.508) (layer "F.Cu") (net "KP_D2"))
 (segment (start 23.9 36.6) (end 23.4 36.1) (width 0.508) (layer "F.Cu") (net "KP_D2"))
 (segment (start 42.8 28) (end 42.8 20) (width 0.508) (layer "F.Cu") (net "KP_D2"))
 (segment (start 37.3 33.9) (end 37.2 33.8) (width 0.508) (layer "F.Cu") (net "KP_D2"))
 (segment (start 38.4 34.7) (end 39.1 34.7) (width 0.508) (layer "F.Cu") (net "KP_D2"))
 (via (at 23.9 36.6) (size 0.6) (drill 0.3) (layers "F.Cu" "B.Cu") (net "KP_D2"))
 (via (at 42.8 38.5) (size 0.6) (drill 0.3) (layers "F.Cu" "B.Cu") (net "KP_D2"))
 (via (at 27.4 33.8) (size 0.6) (drill 0.3) (layers "F.Cu" "B.Cu") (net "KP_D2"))
 (segment (start 42.8 38.5) (end 42.8 46) (width 0.508) (layer "B.Cu") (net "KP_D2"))
 (segment (start 27.4 36.4) (end 26.6 37.2) (width 0.508) (layer "B.Cu") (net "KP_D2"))
 (segment (start 27.4 33.8) (end 27.4 36.4) (width 0.508) (layer "B.Cu") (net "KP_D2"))
 (segment (start 24.5 37.2) (end 23.9 36.6) (width 0.508) (layer "B.Cu") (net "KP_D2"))
 (segment (start 26.6 37.2) (end 24.5 37.2) (width 0.508) (layer "B.Cu") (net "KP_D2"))
 (segment (start 23.4 37.6) (end 23.4 38.6) (width 0.508) (layer "F.Cu") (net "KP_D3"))
 (segment (start 23.2 37.4) (end 23.4 37.6) (width 0.508) (layer "F.Cu") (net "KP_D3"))
 (segment (start 49.4 37.7) (end 49.5 37.8) (width 0.508) (layer "F.Cu") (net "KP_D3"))
 (segment (start 43.7 39.6) (end 45.3 38) (width 0.508) (layer "F.Cu") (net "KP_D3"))
 (segment (start 16.85 37.375) (end 16.8 37.4) (width 0.508) (layer "F.Cu") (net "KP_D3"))
 (segment (start 24.3 39.5) (end 24.5 39.5) (width 0.508) (layer "F.Cu") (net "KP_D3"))
 (segment (start 24.5 39.5) (end 24.6 39.6) (width 0.508) (layer "F.Cu") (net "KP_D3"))
 (segment (start 16.8 37.4) (end 23.2 37.4) (width 0.508) (layer "F.Cu") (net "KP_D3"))
 (segment (start 45.3 28) (end 45.3 20) (width 0.508) (layer "F.Cu") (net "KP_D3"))
 (segment (start 49.5 41.8) (end 45.3 46) (width 0.508) (layer "F.Cu") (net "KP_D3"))
 (segment (start 23.4 38.6) (end 24.3 39.5) (width 0.508) (layer "F.Cu") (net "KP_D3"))
 (segment (start 49.5 37.8) (end 49.5 41.8) (width 0.508) (layer "F.Cu") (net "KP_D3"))
 (segment (start 24.6 39.6) (end 43.7 39.6) (width 0.508) (layer "F.Cu") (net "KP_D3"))
 (segment (start 48.5 36.4) (end 49.4 37.3) (width 0.508) (layer "F.Cu") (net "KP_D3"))
 (segment (start 49.4 37.3) (end 49.4 37.7) (width 0.508) (layer "F.Cu") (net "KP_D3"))
 (segment (start 45.3 38) (end 45.3 28) (width 0.508) (layer "F.Cu") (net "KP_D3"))
 (segment (start 45.3 36.4) (end 48.5 36.4) (width 0.508) (layer "F.Cu") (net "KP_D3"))
 (segment (start 45.2 39.6) (end 44.2 40.6) (width 0.508) (layer "F.Cu") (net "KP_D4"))
 (segment (start 47.9 28) (end 47.86 28) (width 0.508) (layer "F.Cu") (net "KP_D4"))
 (segment (start 16.8 38.6) (end 16.85 38.625) (width 0.508) (layer "F.Cu") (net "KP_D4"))
 (segment (start 47.3 38.6) (end 47 38.6) (width 0.508) (layer "F.Cu") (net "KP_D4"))
 (segment (start 43.9 40.6) (end 43.8 40.7) (width 0.508) (layer "F.Cu") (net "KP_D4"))
 (segment (start 47 38.6) (end 46.1 39.5) (width 0.508) (layer "F.Cu") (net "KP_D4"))
 (segment (start 47.9 35.3) (end 47.9 28) (width 0.508) (layer "F.Cu") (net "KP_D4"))
 (segment (start 47.9 38) (end 47.3 38.6) (width 0.508) (layer "F.Cu") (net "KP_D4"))
 (segment (start 47.9 28) (end 47.9 20) (width 0.508) (layer "F.Cu") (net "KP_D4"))
 (segment (start 44.2 40.6) (end 46.7 43.1) (width 0.508) (layer "F.Cu") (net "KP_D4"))
 (segment (start 44.2 40.6) (end 43.9 40.6) (width 0.508) (layer "F.Cu") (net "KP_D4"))
 (segment (start 45.7 39.6) (end 45.2 39.6) (width 0.508) (layer "F.Cu") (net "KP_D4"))
 (segment (start 46.7 43.1) (end 45.9 43.9) (width 0.508) (layer "F.Cu") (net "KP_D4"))
 (segment (start 45.8 39.5) (end 45.7 39.6) (width 0.508) (layer "F.Cu") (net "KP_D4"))
 (segment (start 18.9 40.7) (end 16.8 38.6) (width 0.508) (layer "F.Cu") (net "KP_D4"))
 (segment (start 47.9 38) (end 47.9 37.5) (width 0.508) (layer "F.Cu") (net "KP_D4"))
 (segment (start 47.86 38) (end 47.9 38) (width 0.508) (layer "F.Cu") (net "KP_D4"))
 (segment (start 43.8 40.7) (end 18.9 40.7) (width 0.508) (layer "F.Cu") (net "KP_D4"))
 (segment (start 46.1 39.5) (end 45.8 39.5) (width 0.508) (layer "F.Cu") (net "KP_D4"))
 (via (at 47.9 37.5) (size 0.6) (drill 0.3) (layers "F.Cu" "B.Cu") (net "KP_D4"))
 (via (at 47.9 35.3) (size 0.6) (drill 0.3) (layers "F.Cu" "B.Cu") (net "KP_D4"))
 (via (at 45.9 43.9) (size 0.6) (drill 0.3) (layers "F.Cu" "B.Cu") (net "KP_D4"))
 (segment (start 45.9 43.9) (end 47.9 45.9) (width 0.508) (layer "B.Cu") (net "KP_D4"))
 (segment (start 47.9 37.5) (end 47.9 35.3) (width 0.508) (layer "B.Cu") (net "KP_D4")))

